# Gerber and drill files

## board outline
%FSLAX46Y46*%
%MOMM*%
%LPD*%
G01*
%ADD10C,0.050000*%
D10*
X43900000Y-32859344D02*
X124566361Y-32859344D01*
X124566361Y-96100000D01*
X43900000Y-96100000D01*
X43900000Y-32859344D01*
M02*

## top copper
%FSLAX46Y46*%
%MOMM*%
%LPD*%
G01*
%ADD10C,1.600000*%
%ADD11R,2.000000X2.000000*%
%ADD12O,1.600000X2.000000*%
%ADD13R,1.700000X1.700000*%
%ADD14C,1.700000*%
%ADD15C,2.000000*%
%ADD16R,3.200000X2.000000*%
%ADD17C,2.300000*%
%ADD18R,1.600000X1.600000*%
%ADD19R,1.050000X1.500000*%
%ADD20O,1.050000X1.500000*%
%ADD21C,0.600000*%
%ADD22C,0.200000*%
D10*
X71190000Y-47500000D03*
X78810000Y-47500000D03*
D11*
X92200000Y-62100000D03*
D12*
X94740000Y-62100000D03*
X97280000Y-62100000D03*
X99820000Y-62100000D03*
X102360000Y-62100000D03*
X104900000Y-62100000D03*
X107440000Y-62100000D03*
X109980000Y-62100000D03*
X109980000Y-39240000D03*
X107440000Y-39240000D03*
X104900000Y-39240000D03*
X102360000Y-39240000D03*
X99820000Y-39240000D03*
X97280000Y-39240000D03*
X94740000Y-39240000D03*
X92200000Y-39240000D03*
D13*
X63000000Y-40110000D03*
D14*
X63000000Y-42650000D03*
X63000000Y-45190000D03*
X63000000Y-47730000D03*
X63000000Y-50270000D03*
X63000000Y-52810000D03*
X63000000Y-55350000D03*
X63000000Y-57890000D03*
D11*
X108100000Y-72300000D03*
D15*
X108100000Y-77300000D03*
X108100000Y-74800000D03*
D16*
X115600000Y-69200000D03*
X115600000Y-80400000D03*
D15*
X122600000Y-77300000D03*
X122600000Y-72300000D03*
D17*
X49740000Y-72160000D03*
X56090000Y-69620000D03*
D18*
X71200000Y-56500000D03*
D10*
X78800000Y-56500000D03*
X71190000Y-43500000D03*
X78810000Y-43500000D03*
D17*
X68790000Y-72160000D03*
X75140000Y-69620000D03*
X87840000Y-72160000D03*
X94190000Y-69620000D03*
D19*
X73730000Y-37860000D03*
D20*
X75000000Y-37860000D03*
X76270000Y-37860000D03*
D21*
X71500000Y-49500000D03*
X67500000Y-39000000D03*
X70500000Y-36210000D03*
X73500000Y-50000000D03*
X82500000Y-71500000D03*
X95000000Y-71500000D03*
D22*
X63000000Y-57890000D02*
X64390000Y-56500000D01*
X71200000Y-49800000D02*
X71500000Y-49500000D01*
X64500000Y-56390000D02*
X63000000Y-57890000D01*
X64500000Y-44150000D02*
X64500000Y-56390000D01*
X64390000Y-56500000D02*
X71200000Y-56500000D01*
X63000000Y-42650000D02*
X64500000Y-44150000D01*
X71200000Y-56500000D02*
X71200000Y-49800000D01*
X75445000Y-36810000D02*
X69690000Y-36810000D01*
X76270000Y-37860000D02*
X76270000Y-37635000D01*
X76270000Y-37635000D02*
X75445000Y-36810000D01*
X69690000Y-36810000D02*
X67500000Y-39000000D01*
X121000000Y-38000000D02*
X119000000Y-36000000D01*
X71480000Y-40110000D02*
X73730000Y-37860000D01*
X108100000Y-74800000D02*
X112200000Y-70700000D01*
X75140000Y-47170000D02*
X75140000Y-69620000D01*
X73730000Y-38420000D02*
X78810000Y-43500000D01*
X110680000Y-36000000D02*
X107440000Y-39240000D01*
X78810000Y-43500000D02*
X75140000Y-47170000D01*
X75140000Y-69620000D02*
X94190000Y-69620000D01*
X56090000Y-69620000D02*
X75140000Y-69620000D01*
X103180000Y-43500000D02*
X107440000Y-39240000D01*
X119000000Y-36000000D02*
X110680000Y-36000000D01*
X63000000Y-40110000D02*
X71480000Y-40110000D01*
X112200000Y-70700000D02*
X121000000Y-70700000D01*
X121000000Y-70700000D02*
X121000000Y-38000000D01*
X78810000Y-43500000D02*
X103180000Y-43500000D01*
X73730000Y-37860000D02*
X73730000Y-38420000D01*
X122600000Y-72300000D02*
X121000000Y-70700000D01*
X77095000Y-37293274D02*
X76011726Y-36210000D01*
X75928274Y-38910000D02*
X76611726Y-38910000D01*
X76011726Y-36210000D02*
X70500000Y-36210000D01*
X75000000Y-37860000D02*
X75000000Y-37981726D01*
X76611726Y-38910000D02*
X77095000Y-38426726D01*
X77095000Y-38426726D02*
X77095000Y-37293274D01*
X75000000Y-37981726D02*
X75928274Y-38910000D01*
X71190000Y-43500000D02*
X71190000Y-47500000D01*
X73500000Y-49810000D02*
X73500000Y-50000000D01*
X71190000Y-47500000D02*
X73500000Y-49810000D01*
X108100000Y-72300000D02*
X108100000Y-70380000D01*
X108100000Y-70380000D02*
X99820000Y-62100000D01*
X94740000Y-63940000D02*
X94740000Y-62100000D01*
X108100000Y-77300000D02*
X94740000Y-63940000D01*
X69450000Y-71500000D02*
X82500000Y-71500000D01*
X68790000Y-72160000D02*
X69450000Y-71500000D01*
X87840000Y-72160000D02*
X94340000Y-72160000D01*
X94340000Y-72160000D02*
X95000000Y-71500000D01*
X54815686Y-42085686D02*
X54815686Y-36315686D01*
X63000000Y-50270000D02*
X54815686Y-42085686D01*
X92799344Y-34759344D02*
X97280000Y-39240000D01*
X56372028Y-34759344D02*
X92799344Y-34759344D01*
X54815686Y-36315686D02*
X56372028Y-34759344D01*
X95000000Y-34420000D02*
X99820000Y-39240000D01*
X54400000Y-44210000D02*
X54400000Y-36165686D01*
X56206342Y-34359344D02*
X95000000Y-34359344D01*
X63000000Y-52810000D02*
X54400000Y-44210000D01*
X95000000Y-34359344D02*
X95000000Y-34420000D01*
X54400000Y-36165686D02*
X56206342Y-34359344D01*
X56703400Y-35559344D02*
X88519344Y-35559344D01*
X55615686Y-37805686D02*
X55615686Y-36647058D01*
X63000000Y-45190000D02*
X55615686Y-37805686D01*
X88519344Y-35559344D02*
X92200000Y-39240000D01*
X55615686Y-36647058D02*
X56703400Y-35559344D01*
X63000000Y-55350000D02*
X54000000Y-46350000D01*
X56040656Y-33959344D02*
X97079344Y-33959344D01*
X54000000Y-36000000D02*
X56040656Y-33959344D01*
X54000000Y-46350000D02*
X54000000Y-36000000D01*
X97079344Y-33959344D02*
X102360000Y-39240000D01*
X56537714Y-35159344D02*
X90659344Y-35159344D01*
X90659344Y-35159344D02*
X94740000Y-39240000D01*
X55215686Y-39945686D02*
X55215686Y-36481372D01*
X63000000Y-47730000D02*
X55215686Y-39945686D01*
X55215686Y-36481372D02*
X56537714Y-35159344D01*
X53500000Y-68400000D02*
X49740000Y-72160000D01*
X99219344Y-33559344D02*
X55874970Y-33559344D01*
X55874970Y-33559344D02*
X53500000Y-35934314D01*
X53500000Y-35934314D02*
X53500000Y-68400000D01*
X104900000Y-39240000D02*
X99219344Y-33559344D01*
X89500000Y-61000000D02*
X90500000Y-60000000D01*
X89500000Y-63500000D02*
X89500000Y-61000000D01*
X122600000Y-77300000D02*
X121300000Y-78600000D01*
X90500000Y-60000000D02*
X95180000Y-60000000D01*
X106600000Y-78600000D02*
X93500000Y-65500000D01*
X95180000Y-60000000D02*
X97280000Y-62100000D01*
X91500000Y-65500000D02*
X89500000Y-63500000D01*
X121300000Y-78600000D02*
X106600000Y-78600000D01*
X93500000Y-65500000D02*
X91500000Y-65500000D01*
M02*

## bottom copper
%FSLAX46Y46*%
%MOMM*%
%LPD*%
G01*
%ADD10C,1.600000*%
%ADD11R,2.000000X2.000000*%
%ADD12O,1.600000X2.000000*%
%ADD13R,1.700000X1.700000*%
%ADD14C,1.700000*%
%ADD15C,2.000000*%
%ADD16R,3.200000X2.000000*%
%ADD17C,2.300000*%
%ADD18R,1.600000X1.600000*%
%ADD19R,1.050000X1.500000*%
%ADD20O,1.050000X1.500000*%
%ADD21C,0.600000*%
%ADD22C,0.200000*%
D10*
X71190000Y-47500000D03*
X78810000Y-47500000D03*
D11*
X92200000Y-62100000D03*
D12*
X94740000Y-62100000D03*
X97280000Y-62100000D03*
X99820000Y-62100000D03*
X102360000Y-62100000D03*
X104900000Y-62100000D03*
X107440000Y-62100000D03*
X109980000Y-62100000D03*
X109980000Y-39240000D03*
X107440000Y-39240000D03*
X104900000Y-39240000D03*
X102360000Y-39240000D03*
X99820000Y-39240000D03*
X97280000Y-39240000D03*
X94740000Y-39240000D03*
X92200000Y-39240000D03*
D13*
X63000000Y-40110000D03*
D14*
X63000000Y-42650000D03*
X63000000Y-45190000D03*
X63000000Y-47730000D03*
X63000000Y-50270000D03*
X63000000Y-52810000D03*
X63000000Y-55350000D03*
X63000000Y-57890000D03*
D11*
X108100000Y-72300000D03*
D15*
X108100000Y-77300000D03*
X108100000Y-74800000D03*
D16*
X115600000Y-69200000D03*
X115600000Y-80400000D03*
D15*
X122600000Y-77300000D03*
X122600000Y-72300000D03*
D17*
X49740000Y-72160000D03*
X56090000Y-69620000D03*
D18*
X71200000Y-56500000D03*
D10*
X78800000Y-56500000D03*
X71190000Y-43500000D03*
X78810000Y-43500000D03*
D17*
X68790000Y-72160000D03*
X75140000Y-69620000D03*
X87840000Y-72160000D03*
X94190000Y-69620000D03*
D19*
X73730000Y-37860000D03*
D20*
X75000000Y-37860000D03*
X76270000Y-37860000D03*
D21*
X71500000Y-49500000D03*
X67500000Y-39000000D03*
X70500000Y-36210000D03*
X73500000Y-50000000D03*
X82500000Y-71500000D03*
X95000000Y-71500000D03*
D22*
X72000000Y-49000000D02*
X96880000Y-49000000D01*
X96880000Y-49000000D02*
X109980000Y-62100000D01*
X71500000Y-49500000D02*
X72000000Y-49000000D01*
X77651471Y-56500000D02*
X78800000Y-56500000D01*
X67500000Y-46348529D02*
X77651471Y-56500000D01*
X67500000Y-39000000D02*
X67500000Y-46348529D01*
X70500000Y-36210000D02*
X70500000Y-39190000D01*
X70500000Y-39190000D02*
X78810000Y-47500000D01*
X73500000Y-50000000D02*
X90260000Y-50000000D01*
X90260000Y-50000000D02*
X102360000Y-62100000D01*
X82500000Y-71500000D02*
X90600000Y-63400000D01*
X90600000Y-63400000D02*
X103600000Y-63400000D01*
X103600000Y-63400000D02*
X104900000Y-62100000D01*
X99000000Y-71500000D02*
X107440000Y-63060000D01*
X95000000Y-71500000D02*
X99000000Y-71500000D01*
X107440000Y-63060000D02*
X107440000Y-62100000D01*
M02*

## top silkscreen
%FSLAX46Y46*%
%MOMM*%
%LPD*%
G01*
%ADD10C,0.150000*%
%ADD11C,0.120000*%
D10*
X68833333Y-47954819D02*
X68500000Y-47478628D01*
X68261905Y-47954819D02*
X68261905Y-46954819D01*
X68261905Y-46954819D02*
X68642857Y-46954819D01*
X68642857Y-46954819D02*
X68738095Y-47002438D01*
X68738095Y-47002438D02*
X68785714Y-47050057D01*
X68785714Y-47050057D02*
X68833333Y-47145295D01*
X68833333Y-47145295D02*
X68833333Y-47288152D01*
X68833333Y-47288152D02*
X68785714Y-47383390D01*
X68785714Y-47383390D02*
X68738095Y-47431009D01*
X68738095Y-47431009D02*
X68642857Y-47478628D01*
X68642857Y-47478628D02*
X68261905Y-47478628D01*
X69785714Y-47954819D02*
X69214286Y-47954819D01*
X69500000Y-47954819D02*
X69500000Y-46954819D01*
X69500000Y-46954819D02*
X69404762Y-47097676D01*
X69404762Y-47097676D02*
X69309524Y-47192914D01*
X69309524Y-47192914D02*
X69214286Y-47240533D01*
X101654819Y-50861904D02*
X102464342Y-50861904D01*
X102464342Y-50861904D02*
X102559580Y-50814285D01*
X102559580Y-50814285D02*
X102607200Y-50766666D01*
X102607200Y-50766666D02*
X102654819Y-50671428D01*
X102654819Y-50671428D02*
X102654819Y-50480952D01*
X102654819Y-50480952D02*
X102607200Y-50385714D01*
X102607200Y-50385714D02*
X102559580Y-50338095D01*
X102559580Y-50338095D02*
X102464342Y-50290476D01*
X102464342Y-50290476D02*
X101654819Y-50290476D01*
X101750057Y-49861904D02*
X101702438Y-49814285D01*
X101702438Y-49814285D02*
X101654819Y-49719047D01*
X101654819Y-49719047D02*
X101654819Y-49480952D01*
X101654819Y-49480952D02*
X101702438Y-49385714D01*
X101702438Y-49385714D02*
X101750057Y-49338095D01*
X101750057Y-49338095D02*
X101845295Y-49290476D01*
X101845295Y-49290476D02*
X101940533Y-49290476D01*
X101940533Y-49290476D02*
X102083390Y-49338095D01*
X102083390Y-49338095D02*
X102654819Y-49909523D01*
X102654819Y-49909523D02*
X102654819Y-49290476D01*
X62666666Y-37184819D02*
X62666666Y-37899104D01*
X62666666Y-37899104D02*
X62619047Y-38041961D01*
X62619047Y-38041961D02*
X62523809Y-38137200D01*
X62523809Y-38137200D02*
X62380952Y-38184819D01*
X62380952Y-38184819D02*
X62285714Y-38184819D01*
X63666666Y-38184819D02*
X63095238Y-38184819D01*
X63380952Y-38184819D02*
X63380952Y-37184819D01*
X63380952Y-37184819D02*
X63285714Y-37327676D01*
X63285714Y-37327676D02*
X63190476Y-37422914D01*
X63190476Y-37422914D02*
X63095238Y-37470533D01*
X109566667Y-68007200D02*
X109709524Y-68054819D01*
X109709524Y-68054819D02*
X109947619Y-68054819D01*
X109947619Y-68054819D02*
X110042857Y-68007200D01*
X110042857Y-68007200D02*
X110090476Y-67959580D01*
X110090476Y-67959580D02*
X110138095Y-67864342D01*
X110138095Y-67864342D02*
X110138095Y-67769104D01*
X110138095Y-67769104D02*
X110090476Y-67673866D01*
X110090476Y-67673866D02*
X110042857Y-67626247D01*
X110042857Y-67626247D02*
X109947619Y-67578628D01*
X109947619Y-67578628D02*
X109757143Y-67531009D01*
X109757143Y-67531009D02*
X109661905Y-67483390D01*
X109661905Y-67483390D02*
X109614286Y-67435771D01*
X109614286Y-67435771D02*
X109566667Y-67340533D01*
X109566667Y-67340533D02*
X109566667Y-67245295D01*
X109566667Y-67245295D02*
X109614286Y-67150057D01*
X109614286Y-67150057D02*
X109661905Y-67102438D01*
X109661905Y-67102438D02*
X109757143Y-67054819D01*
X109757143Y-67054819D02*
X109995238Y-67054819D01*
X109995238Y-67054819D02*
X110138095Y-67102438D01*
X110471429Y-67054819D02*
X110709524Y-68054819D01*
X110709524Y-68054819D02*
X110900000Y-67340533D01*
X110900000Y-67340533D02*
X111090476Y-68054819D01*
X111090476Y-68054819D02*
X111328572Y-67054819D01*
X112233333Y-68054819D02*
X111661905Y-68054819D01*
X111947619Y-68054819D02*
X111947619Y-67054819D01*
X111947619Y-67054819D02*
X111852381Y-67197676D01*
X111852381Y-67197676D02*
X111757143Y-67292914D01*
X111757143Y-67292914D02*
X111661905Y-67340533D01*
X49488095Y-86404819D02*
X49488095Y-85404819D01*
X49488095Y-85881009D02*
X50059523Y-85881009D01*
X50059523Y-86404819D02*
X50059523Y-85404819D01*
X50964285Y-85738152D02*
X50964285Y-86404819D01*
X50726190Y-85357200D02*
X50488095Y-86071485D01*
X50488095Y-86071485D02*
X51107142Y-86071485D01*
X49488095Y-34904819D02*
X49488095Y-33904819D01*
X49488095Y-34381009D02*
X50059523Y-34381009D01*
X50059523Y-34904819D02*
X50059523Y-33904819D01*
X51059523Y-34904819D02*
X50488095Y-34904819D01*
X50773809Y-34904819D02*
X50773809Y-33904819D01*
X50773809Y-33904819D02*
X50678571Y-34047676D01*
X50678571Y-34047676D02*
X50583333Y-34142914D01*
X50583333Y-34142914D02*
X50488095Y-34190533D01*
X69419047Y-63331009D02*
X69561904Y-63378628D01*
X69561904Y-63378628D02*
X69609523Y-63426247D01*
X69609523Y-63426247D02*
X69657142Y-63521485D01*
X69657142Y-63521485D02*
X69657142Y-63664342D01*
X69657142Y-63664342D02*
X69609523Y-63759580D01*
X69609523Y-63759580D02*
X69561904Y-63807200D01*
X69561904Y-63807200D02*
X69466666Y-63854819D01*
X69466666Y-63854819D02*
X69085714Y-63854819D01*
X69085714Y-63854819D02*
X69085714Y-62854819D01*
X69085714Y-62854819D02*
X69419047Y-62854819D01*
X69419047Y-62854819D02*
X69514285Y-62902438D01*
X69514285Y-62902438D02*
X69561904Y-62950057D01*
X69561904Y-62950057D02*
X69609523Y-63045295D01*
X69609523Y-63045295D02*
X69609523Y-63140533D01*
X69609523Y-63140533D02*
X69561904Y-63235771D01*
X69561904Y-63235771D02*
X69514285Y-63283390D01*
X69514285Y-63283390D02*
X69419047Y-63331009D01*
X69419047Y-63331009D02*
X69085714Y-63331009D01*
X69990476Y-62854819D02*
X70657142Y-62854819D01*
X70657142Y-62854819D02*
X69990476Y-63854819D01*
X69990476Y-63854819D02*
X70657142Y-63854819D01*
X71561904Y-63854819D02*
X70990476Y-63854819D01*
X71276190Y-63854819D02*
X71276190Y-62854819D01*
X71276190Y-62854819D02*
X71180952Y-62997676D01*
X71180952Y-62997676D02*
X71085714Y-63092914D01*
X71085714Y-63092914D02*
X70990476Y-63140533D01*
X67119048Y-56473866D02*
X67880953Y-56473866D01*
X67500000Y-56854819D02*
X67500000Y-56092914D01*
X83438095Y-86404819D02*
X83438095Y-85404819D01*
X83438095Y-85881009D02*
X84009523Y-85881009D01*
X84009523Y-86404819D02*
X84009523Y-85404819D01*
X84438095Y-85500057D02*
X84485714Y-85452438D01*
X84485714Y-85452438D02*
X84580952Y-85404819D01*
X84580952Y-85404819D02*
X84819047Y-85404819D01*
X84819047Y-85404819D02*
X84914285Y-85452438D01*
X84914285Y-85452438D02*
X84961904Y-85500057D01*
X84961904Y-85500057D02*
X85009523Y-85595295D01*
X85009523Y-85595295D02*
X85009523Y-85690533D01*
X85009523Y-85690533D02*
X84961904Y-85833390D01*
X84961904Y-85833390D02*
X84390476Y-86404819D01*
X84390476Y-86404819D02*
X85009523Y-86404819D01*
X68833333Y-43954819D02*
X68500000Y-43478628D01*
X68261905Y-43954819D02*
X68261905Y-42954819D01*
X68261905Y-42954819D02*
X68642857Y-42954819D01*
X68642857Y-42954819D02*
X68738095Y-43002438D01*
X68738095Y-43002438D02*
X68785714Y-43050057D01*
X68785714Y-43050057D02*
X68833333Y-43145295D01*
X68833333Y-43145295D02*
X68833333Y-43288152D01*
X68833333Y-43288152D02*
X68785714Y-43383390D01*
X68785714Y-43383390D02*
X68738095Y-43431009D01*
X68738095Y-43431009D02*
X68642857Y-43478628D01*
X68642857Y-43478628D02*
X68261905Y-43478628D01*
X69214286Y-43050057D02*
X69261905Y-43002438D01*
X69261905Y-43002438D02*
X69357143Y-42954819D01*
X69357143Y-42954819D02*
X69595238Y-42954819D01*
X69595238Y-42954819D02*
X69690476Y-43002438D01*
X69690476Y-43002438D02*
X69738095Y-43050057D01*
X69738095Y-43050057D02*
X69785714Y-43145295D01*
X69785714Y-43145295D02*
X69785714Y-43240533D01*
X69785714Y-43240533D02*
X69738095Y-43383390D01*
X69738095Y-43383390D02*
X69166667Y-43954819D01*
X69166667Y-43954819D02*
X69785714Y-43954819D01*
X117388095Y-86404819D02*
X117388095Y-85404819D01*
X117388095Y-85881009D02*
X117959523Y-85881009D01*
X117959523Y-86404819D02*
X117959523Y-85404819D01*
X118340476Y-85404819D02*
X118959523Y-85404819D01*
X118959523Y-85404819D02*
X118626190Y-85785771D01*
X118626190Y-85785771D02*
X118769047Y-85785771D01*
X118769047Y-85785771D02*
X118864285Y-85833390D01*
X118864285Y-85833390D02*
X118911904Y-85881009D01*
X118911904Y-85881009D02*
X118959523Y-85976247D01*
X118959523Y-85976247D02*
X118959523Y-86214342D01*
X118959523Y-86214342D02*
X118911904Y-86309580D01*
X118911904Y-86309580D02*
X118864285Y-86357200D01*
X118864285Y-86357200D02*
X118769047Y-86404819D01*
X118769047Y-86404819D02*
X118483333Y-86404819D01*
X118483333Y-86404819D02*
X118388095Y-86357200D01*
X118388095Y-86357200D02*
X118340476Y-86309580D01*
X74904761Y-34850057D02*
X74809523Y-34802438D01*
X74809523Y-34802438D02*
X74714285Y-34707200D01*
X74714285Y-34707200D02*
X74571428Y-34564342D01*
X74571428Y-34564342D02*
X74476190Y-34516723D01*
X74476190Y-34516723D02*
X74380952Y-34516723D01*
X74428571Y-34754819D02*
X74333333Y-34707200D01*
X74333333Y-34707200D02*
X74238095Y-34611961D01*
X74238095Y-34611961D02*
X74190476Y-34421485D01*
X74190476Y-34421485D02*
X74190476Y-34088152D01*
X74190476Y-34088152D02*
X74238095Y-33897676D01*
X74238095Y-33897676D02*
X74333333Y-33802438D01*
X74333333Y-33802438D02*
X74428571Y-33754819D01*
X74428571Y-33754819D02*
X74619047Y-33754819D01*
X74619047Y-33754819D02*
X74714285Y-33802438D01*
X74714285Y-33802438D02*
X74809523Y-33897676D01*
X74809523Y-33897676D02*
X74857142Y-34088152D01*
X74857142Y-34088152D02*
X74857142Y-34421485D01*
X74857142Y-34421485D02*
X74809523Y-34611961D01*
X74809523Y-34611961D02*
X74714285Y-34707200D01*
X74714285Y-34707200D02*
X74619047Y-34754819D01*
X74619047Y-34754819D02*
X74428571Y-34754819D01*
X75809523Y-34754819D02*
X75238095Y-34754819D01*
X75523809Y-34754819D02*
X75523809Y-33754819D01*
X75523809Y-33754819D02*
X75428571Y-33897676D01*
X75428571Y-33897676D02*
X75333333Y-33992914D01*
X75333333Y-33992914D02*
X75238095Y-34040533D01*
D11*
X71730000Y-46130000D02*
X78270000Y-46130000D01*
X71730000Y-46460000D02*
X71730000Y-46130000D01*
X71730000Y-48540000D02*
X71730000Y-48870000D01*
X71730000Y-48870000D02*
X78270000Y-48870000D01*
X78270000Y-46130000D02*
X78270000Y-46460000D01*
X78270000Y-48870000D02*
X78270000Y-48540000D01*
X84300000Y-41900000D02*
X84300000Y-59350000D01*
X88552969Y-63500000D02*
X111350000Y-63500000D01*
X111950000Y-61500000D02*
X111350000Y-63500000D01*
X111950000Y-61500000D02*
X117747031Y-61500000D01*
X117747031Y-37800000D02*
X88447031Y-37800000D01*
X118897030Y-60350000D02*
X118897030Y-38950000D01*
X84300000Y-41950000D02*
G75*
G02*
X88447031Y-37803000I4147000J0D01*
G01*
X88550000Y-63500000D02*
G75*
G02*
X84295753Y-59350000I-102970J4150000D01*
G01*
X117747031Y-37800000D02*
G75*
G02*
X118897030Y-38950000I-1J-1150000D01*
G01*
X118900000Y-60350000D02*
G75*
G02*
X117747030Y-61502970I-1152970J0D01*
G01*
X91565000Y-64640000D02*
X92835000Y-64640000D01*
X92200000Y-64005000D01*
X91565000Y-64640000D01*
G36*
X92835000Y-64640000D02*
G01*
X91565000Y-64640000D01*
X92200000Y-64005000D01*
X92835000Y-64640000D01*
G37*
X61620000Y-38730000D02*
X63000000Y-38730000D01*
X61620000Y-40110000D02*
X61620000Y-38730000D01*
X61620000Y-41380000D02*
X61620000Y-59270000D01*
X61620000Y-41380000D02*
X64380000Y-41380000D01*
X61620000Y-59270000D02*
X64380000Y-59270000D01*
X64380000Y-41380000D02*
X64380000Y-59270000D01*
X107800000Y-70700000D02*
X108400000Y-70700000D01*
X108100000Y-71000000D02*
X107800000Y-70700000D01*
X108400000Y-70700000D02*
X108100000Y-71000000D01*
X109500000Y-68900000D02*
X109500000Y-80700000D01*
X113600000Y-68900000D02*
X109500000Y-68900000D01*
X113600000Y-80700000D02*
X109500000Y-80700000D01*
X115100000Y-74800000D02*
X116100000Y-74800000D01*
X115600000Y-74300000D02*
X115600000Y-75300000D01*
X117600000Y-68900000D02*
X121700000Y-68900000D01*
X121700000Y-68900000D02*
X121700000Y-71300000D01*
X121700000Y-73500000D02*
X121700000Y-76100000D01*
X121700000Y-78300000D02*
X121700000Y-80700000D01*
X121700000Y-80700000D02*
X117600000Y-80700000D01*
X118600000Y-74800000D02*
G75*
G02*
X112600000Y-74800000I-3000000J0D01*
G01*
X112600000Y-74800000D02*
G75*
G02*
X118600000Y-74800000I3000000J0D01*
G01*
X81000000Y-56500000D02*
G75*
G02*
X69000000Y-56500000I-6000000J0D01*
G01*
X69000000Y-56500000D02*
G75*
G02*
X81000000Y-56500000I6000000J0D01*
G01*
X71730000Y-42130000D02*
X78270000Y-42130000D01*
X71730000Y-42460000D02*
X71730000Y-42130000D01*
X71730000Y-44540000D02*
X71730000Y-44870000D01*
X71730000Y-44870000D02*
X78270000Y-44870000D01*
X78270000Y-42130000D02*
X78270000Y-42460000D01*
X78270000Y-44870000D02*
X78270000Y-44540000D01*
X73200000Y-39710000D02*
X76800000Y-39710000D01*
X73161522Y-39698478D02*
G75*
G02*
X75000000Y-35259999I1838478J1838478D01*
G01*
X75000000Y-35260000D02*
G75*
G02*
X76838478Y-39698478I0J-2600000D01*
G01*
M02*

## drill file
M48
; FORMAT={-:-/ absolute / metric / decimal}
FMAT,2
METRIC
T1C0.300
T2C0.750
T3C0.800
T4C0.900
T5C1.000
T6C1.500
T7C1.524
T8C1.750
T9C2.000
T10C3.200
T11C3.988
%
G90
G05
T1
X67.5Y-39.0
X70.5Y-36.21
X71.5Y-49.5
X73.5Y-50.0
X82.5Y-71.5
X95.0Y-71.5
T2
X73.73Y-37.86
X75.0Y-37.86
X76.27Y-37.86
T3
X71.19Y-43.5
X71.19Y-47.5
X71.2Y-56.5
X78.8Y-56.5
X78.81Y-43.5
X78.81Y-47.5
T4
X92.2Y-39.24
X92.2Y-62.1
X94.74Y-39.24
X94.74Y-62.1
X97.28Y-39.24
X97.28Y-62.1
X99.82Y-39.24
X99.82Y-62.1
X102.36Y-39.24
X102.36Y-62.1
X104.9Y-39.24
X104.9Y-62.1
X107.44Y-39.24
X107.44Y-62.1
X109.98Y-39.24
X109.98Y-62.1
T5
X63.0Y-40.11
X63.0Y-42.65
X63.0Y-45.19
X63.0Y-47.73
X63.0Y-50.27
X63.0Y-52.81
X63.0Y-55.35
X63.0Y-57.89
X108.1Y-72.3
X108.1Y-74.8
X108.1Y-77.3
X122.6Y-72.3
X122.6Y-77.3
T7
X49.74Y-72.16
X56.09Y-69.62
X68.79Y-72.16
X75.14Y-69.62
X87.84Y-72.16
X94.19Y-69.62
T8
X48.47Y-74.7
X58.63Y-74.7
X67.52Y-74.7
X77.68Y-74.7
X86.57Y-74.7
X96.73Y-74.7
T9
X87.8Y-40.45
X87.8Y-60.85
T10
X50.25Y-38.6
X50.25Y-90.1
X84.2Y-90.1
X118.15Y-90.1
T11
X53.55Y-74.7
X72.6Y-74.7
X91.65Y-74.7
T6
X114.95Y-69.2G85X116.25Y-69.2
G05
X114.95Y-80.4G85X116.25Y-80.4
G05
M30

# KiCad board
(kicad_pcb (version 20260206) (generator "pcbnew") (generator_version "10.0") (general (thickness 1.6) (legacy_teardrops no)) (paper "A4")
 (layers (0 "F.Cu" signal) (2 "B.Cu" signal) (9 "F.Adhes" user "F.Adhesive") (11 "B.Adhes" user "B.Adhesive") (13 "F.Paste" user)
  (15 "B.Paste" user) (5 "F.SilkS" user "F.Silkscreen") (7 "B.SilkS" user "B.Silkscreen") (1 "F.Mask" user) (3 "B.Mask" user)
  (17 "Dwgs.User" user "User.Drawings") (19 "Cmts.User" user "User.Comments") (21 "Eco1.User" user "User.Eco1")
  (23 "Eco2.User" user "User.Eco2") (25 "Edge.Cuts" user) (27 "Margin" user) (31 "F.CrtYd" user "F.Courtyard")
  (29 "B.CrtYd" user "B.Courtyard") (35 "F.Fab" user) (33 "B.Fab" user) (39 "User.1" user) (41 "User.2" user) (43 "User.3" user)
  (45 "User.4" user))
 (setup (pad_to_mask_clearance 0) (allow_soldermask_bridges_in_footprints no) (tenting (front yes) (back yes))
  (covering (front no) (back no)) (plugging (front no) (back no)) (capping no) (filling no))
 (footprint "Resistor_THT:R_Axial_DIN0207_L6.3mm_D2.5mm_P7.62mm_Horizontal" (layer "F.Cu") (at 71.19 47.5)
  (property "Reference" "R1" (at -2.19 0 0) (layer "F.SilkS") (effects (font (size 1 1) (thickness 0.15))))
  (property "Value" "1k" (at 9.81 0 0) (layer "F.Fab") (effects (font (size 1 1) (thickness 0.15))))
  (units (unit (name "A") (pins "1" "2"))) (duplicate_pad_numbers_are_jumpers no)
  (fp_line (start 0.54 -1.37) (end 7.08 -1.37) (stroke (width 0.12) (type solid)) (layer "F.SilkS"))
  (fp_line (start 0.54 -1.04) (end 0.54 -1.37) (stroke (width 0.12) (type solid)) (layer "F.SilkS"))
  (fp_line (start 0.54 1.04) (end 0.54 1.37) (stroke (width 0.12) (type solid)) (layer "F.SilkS"))
  (fp_line (start 0.54 1.37) (end 7.08 1.37) (stroke (width 0.12) (type solid)) (layer "F.SilkS"))
  (fp_line (start 7.08 -1.37) (end 7.08 -1.04) (stroke (width 0.12) (type solid)) (layer "F.SilkS"))
  (fp_line (start 7.08 1.37) (end 7.08 1.04) (stroke (width 0.12) (type solid)) (layer "F.SilkS"))
  (pad "1" thru_hole circle (at 0 0) (size 1.6 1.6) (drill 0.8) (layers "*.Cu" "*.Mask") (remove_unused_layers no) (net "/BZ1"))
  (pad "2" thru_hole circle (at 7.62 0) (size 1.6 1.6) (drill 0.8) (layers "*.Cu" "*.Mask") (remove_unused_layers no) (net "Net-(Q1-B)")))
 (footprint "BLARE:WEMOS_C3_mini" (layer "F.Cu") (at 92.2 62.1 90)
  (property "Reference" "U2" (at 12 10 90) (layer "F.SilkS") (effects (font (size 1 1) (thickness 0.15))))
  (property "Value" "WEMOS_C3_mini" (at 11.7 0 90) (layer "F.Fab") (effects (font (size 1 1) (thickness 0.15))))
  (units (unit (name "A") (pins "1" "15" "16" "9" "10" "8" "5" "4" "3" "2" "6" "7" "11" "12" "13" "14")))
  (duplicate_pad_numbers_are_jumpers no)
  (fp_line (start 20.2 -7.9) (end 2.75 -7.9) (stroke (width 0.12) (type solid)) (layer "F.SilkS"))
  (fp_line (start -1.4 -3.647031) (end -1.4 19.15) (stroke (width 0.12) (type solid)) (layer "F.SilkS"))
  (fp_line (start 0.6 19.75) (end -1.4 19.15) (stroke (width 0.12) (type default)) (layer "F.SilkS"))
  (fp_line (start 0.6 19.75) (end 0.6 25.547031) (stroke (width 0.12) (type solid)) (layer "F.SilkS"))
  (fp_line (start 24.3 25.547031) (end 24.3 -3.752969) (stroke (width 0.12) (type solid)) (layer "F.SilkS"))
  (fp_line (start 1.75 26.69703) (end 23.15 26.69703) (stroke (width 0.12) (type solid)) (layer "F.SilkS"))
  (fp_arc (start 20.15 -7.9) (mid 23.082383 -6.685361) (end 24.297 -3.752969) (stroke (width 0.12) (type solid)) (layer "F.SilkS"))
  (fp_arc (start -1.4 -3.65) (mid -0.221578 -6.651732) (end 2.75 -7.904246) (stroke (width 0.12) (type solid)) (layer "F.SilkS"))
  (fp_arc (start 24.3 25.547031) (mid 23.963172 26.360203) (end 23.15 26.69703) (stroke (width 0.12) (type solid)) (layer "F.SilkS"))
  (fp_arc (start 1.75 26.7) (mid 0.934727 26.362303) (end 0.59703 25.54703) (stroke (width 0.12) (type solid)) (layer "F.SilkS"))
  (fp_poly (pts (xy -2.54 -0.635) (xy -2.54 0.635) (xy -1.905 0)) (stroke (width 0.12) (type solid)) (fill yes) (layer "F.SilkS"))
  (pad "" np_thru_hole circle (at 1.25 -4.4 90) (size 3 3) (drill 2) (layers "*.Mask"))
  (pad "" np_thru_hole circle (at 21.65 -4.4 90) (size 3 3) (drill 2) (layers "*.Mask"))
  (pad "1" thru_hole rect (at 0 0 90) (size 2 2) (drill 0.9) (layers "*.Cu" "*.Mask") (remove_unused_layers no)
   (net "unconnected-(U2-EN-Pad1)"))
  (pad "2" thru_hole oval (at 0 2.54 90) (size 2 1.6) (drill 0.9) (layers "*.Cu" "*.Mask") (remove_unused_layers no) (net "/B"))
  (pad "3" thru_hole oval (at 0 5.08 90) (size 2 1.6) (drill 0.9) (layers "*.Cu" "*.Mask") (remove_unused_layers no) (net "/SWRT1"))
  (pad "4" thru_hole oval (at 0 7.62 90) (size 2 1.6) (drill 0.9) (layers "*.Cu" "*.Mask") (remove_unused_layers no) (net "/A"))
  (pad "5" thru_hole oval (at 0 10.16 90) (size 2 1.6) (drill 0.9) (layers "*.Cu" "*.Mask") (remove_unused_layers no) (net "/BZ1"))
  (pad "6" thru_hole oval (at 0 12.7 90) (size 2 1.6) (drill 0.9) (layers "*.Cu" "*.Mask") (remove_unused_layers no) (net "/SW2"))
  (pad "7" thru_hole oval (at 0 15.24 90) (size 2 1.6) (drill 0.9) (layers "*.Cu" "*.Mask") (remove_unused_layers no) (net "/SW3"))
  (pad "8" thru_hole oval (at 0 17.78 90) (size 2 1.6) (drill 0.9) (layers "*.Cu" "*.Mask") (remove_unused_layers no) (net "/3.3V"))
  (pad "9" thru_hole oval (at 22.86 17.78 90) (size 2 1.6) (drill 0.9) (layers "*.Cu" "*.Mask") (remove_unused_layers no)
   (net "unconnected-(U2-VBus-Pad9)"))
  (pad "10" thru_hole oval (at 22.86 15.24 90) (size 2 1.6) (drill 0.9) (layers "*.Cu" "*.Mask") (remove_unused_layers no) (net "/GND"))
  (pad "11" thru_hole oval (at 22.86 12.7 90) (size 2 1.6) (drill 0.9) (layers "*.Cu" "*.Mask") (remove_unused_layers no) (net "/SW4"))
  (pad "12" thru_hole oval (at 22.86 10.16 90) (size 2 1.6) (drill 0.9) (layers "*.Cu" "*.Mask") (remove_unused_layers no) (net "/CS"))
  (pad "13" thru_hole oval (at 22.86 7.62 90) (size 2 1.6) (drill 0.9) (layers "*.Cu" "*.Mask") (remove_unused_layers no) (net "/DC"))
  (pad "14" thru_hole oval (at 22.86 5.08 90) (size 2 1.6) (drill 0.9) (layers "*.Cu" "*.Mask") (remove_unused_layers no) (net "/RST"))
  (pad "15" thru_hole oval (at 22.86 2.54 90) (size 2 1.6) (drill 0.9) (layers "*.Cu" "*.Mask") (remove_unused_layers no) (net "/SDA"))
  (pad "16" thru_hole oval (at 22.86 0 90) (size 2 1.6) (drill 0.9) (layers "*.Cu" "*.Mask") (remove_unused_layers no) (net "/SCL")))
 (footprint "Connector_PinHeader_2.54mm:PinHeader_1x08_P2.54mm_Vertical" (layer "F.Cu") (at 63 40.11)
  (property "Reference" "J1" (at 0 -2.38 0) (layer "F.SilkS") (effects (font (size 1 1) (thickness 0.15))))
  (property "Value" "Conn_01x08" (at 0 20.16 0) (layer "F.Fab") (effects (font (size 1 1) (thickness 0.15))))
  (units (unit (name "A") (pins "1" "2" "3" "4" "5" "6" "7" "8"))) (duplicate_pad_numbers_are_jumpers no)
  (fp_line (start -1.38 -1.38) (end 0 -1.38) (stroke (width 0.12) (type solid)) (layer "F.SilkS"))
  (fp_line (start -1.38 0) (end -1.38 -1.38) (stroke (width 0.12) (type solid)) (layer "F.SilkS"))
  (fp_line (start -1.38 1.27) (end -1.38 19.16) (stroke (width 0.12) (type solid)) (layer "F.SilkS"))
  (fp_line (start -1.38 1.27) (end 1.38 1.27) (stroke (width 0.12) (type solid)) (layer "F.SilkS"))
  (fp_line (start -1.38 19.16) (end 1.38 19.16) (stroke (width 0.12) (type solid)) (layer "F.SilkS"))
  (fp_line (start 1.38 1.27) (end 1.38 19.16) (stroke (width 0.12) (type solid)) (layer "F.SilkS"))
  (pad "1" thru_hole rect (at 0 0) (size 1.7 1.7) (drill 1) (layers "*.Cu" "*.Mask") (remove_unused_layers no) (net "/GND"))
  (pad "2" thru_hole circle (at 0 2.54) (size 1.7 1.7) (drill 1) (layers "*.Cu" "*.Mask") (remove_unused_layers no) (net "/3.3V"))
  (pad "3" thru_hole circle (at 0 5.08) (size 1.7 1.7) (drill 1) (layers "*.Cu" "*.Mask") (remove_unused_layers no) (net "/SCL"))
  (pad "4" thru_hole circle (at 0 7.62) (size 1.7 1.7) (drill 1) (layers "*.Cu" "*.Mask") (remove_unused_layers no) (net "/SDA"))
  (pad "5" thru_hole circle (at 0 10.16) (size 1.7 1.7) (drill 1) (layers "*.Cu" "*.Mask") (remove_unused_layers no) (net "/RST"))
  (pad "6" thru_hole circle (at 0 12.7) (size 1.7 1.7) (drill 1) (layers "*.Cu" "*.Mask") (remove_unused_layers no) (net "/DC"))
  (pad "7" thru_hole circle (at 0 15.24) (size 1.7 1.7) (drill 1) (layers "*.Cu" "*.Mask") (remove_unused_layers no) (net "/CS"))
  (pad "8" thru_hole circle (at 0 17.78) (size 1.7 1.7) (drill 1) (layers "*.Cu" "*.Mask") (remove_unused_layers no) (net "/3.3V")))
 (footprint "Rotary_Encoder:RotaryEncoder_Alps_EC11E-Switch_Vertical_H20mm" (layer "F.Cu") (at 108.1 72.3)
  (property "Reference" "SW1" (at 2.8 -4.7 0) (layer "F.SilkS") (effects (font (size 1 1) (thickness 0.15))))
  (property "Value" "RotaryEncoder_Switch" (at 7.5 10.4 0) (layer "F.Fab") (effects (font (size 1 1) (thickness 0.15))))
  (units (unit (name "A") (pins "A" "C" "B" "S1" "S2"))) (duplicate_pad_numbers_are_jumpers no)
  (fp_line (start -0.3 -1.6) (end 0.3 -1.6) (stroke (width 0.12) (type solid)) (layer "F.SilkS"))
  (fp_line (start 0 -1.3) (end -0.3 -1.6) (stroke (width 0.12) (type solid)) (layer "F.SilkS"))
  (fp_line (start 0.3 -1.6) (end 0 -1.3) (stroke (width 0.12) (type solid)) (layer "F.SilkS"))
  (fp_line (start 1.4 -3.4) (end 1.4 8.4) (stroke (width 0.12) (type solid)) (layer "F.SilkS"))
  (fp_line (start 5.5 -3.4) (end 1.4 -3.4) (stroke (width 0.12) (type solid)) (layer "F.SilkS"))
  (fp_line (start 5.5 8.4) (end 1.4 8.4) (stroke (width 0.12) (type solid)) (layer "F.SilkS"))
  (fp_line (start 7 2.5) (end 8 2.5) (stroke (width 0.12) (type solid)) (layer "F.SilkS"))
  (fp_line (start 7.5 2) (end 7.5 3) (stroke (width 0.12) (type solid)) (layer "F.SilkS"))
  (fp_line (start 9.5 -3.4) (end 13.6 -3.4) (stroke (width 0.12) (type solid)) (layer "F.SilkS"))
  (fp_line (start 13.6 -3.4) (end 13.6 -1) (stroke (width 0.12) (type solid)) (layer "F.SilkS"))
  (fp_line (start 13.6 1.2) (end 13.6 3.8) (stroke (width 0.12) (type solid)) (layer "F.SilkS"))
  (fp_line (start 13.6 6) (end 13.6 8.4) (stroke (width 0.12) (type solid)) (layer "F.SilkS"))
  (fp_line (start 13.6 8.4) (end 9.5 8.4) (stroke (width 0.12) (type solid)) (layer "F.SilkS"))
  (fp_circle (center 7.5 2.5) (end 10.5 2.5) (stroke (width 0.12) (type solid)) (fill no) (layer "F.SilkS"))
  (pad "A" thru_hole rect (at 0 0) (size 2 2) (drill 1) (layers "*.Cu" "*.Mask") (remove_unused_layers no) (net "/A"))
  (pad "B" thru_hole circle (at 0 5) (size 2 2) (drill 1) (layers "*.Cu" "*.Mask") (remove_unused_layers no) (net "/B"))
  (pad "C" thru_hole circle (at 0 2.5) (size 2 2) (drill 1) (layers "*.Cu" "*.Mask") (remove_unused_layers no) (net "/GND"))
  (pad "MP" thru_hole rect (at 7.5 -3.1) (size 3.2 2) (drill oval 2.8 1.5) (layers "*.Cu" "*.Mask") (remove_unused_layers no))
  (pad "MP" thru_hole rect (at 7.5 8.1) (size 3.2 2) (drill oval 2.8 1.5) (layers "*.Cu" "*.Mask") (remove_unused_layers no))
  (pad "S1" thru_hole circle (at 14.5 5) (size 2 2) (drill 1) (layers "*.Cu" "*.Mask") (remove_unused_layers no) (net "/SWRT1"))
  (pad "S2" thru_hole circle (at 14.5 0) (size 2 2) (drill 1) (layers "*.Cu" "*.Mask") (remove_unused_layers no) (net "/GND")))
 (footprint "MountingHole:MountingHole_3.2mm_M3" (layer "F.Cu") (at 50.25 90.1)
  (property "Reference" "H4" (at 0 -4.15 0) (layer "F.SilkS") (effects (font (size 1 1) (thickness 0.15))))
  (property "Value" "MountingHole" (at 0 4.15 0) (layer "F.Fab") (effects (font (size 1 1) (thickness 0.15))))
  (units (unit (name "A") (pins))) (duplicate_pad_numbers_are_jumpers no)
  (pad "" np_thru_hole circle (at 0 0) (size 3.2 3.2) (drill 3.2) (layers "*.Cu" "*.Mask")))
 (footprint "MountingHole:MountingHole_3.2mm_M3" (layer "F.Cu") (at 50.25 38.6)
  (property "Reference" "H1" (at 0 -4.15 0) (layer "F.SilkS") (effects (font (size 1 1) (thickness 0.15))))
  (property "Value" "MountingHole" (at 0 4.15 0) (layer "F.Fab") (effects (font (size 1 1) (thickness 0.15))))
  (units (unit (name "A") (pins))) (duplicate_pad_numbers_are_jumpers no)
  (pad "" np_thru_hole circle (at 0 0) (size 3.2 3.2) (drill 3.2) (layers "*.Cu" "*.Mask")))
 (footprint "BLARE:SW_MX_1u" (layer "F.Cu") (at 53.55 74.7)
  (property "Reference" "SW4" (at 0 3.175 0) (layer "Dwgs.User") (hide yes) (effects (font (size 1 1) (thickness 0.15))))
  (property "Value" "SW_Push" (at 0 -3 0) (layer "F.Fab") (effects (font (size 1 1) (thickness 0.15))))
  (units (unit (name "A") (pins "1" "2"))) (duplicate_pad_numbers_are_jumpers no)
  (pad "" np_thru_hole circle (at -5.08 0) (size 1.75 1.75) (drill 1.75) (layers "*.Cu" "*.Mask"))
  (pad "" np_thru_hole circle (at 0 0) (size 3.9878 3.9878) (drill 3.9878) (layers "*.Cu" "*.Mask"))
  (pad "" np_thru_hole circle (at 5.08 0) (size 1.75 1.75) (drill 1.75) (layers "*.Cu" "*.Mask"))
  (pad "1" thru_hole circle (at -3.81 -2.54) (size 2.3 2.3) (drill 1.524) (layers "*.Cu" "B.Mask") (remove_unused_layers no) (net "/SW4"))
  (pad "2" thru_hole circle (at 2.54 -5.08) (size 2.3 2.3) (drill 1.524) (layers "*.Cu" "B.Mask") (remove_unused_layers no) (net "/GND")))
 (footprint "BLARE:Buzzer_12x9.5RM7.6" (layer "F.Cu") (at 75 56.5)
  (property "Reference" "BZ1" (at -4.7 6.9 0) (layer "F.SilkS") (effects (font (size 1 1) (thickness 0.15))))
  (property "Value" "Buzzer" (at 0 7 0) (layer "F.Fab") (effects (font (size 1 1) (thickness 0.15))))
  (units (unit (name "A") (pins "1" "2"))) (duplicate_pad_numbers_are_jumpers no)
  (fp_circle (center 0 0) (end 6 0) (stroke (width 0.12) (type solid)) (fill no) (layer "F.SilkS"))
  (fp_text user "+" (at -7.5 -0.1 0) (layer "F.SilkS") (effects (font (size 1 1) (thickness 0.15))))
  (pad "1" thru_hole rect (at -3.8 0) (size 1.6 1.6) (drill 0.8) (layers "*.Cu" "*.Mask") (remove_unused_layers no) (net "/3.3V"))
  (pad "2" thru_hole circle (at 3.8 0) (size 1.6 1.6) (drill 0.8) (layers "*.Cu" "*.Mask") (remove_unused_layers no) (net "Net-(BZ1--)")))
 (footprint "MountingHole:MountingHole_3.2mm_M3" (layer "F.Cu") (at 84.2 90.1)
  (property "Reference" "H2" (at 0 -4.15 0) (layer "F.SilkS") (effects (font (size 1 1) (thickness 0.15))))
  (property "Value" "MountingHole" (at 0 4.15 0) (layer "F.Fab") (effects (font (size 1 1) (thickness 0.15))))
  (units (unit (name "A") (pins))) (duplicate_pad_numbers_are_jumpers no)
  (pad "" np_thru_hole circle (at 0 0) (size 3.2 3.2) (drill 3.2) (layers "*.Cu" "*.Mask")))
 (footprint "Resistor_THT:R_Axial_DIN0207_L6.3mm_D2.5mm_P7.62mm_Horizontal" (layer "F.Cu") (at 71.19 43.5)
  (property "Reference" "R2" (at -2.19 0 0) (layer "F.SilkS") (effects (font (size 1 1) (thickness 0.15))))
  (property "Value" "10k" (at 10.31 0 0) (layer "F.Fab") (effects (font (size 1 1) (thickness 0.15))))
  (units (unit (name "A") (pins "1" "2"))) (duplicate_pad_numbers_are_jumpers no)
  (fp_line (start 0.54 -1.37) (end 7.08 -1.37) (stroke (width 0.12) (type solid)) (layer "F.SilkS"))
  (fp_line (start 0.54 -1.04) (end 0.54 -1.37) (stroke (width 0.12) (type solid)) (layer "F.SilkS"))
  (fp_line (start 0.54 1.04) (end 0.54 1.37) (stroke (width 0.12) (type solid)) (layer "F.SilkS"))
  (fp_line (start 0.54 1.37) (end 7.08 1.37) (stroke (width 0.12) (type solid)) (layer "F.SilkS"))
  (fp_line (start 7.08 -1.37) (end 7.08 -1.04) (stroke (width 0.12) (type solid)) (layer "F.SilkS"))
  (fp_line (start 7.08 1.37) (end 7.08 1.04) (stroke (width 0.12) (type solid)) (layer "F.SilkS"))
  (pad "1" thru_hole circle (at 0 0) (size 1.6 1.6) (drill 0.8) (layers "*.Cu" "*.Mask") (remove_unused_layers no) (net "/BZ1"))
  (pad "2" thru_hole circle (at 7.62 0) (size 1.6 1.6) (drill 0.8) (layers "*.Cu" "*.Mask") (remove_unused_layers no) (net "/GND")))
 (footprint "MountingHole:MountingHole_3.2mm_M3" (layer "F.Cu") (at 118.15 90.1)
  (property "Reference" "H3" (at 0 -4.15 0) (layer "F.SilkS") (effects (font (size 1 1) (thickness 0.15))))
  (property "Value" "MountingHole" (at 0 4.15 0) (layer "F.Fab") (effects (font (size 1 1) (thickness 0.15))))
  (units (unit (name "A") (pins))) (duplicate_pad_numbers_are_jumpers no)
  (pad "" np_thru_hole circle (at 0 0) (size 3.2 3.2) (drill 3.2) (layers "*.Cu" "*.Mask")))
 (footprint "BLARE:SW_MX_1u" (layer "F.Cu") (at 72.6 74.7)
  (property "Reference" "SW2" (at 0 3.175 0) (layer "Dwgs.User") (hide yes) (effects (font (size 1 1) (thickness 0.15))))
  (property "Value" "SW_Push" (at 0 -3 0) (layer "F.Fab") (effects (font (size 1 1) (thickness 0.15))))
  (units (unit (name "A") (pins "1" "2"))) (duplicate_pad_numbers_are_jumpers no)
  (pad "" np_thru_hole circle (at -5.08 0) (size 1.75 1.75) (drill 1.75) (layers "*.Cu" "*.Mask"))
  (pad "" np_thru_hole circle (at 0 0) (size 3.9878 3.9878) (drill 3.9878) (layers "*.Cu" "*.Mask"))
  (pad "" np_thru_hole circle (at 5.08 0) (size 1.75 1.75) (drill 1.75) (layers "*.Cu" "*.Mask"))
  (pad "1" thru_hole circle (at -3.81 -2.54) (size 2.3 2.3) (drill 1.524) (layers "*.Cu" "B.Mask") (remove_unused_layers no) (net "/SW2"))
  (pad "2" thru_hole circle (at 2.54 -5.08) (size 2.3 2.3) (drill 1.524) (layers "*.Cu" "B.Mask") (remove_unused_layers no) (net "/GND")))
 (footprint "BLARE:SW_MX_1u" (layer "F.Cu") (at 91.65 74.7)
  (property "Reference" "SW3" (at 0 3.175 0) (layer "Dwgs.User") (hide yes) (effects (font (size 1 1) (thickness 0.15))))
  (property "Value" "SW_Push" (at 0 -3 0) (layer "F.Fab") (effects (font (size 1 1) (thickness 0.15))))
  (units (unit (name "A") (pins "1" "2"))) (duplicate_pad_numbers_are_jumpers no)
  (pad "" np_thru_hole circle (at -5.08 0) (size 1.75 1.75) (drill 1.75) (layers "*.Cu" "*.Mask"))
  (pad "" np_thru_hole circle (at 0 0) (size 3.9878 3.9878) (drill 3.9878) (layers "*.Cu" "*.Mask"))
  (pad "" np_thru_hole circle (at 5.08 0) (size 1.75 1.75) (drill 1.75) (layers "*.Cu" "*.Mask"))
  (pad "1" thru_hole circle (at -3.81 -2.54) (size 2.3 2.3) (drill 1.524) (layers "*.Cu" "B.Mask") (remove_unused_layers no) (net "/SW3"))
  (pad "2" thru_hole circle (at 2.54 -5.08) (size 2.3 2.3) (drill 1.524) (layers "*.Cu" "B.Mask") (remove_unused_layers no) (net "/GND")))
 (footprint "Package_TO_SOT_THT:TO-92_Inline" (layer "F.Cu") (at 73.73 37.86)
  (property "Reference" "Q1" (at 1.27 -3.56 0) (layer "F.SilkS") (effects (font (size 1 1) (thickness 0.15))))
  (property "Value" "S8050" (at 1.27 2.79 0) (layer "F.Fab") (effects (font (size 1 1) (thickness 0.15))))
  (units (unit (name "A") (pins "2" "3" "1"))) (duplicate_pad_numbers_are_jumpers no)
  (fp_line (start -0.53 1.85) (end 3.07 1.85) (stroke (width 0.12) (type solid)) (layer "F.SilkS"))
  (fp_arc (start -0.568478 1.838478) (mid -1.132087 -0.994977) (end 1.27 -2.6) (stroke (width 0.12) (type solid)) (layer "F.SilkS"))
  (fp_arc (start 1.27 -2.6) (mid 3.672087 -0.994977) (end 3.108478 1.838478) (stroke (width 0.12) (type solid)) (layer "F.SilkS"))
  (pad "1" thru_hole rect (at 0 0) (size 1.05 1.5) (drill 0.75) (layers "*.Cu" "*.Mask") (remove_unused_layers no) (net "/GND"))
  (pad "2" thru_hole oval (at 1.27 0) (size 1.05 1.5) (drill 0.75) (layers "*.Cu" "*.Mask") (remove_unused_layers no) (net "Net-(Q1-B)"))
  (pad "3" thru_hole oval (at 2.54 0) (size 1.05 1.5) (drill 0.75) (layers "*.Cu" "*.Mask") (remove_unused_layers no) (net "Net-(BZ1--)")))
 (gr_rect (start 43.9 32.859344) (end 124.566361 96.1) (stroke (width 0.05) (type default)) (fill no) (layer "Edge.Cuts"))
 (segment (start 63 57.89) (end 64.39 56.5) (width 0.2) (layer "F.Cu") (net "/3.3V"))
 (segment (start 71.2 49.8) (end 71.5 49.5) (width 0.2) (layer "F.Cu") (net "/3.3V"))
 (segment (start 64.5 56.39) (end 63 57.89) (width 0.2) (layer "F.Cu") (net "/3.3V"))
 (segment (start 64.5 44.15) (end 64.5 56.39) (width 0.2) (layer "F.Cu") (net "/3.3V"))
 (segment (start 64.39 56.5) (end 71.2 56.5) (width 0.2) (layer "F.Cu") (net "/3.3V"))
 (segment (start 63 42.65) (end 64.5 44.15) (width 0.2) (layer "F.Cu") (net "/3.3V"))
 (segment (start 71.2 56.5) (end 71.2 49.8) (width 0.2) (layer "F.Cu") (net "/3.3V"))
 (via (at 71.5 49.5) (size 0.6) (drill 0.3) (layers "F.Cu" "B.Cu") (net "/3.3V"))
 (segment (start 72 49) (end 96.88 49) (width 0.2) (layer "B.Cu") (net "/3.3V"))
 (segment (start 96.88 49) (end 109.98 62.1) (width 0.2) (layer "B.Cu") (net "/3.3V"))
 (segment (start 71.5 49.5) (end 72 49) (width 0.2) (layer "B.Cu") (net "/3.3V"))
 (segment (start 75.445 36.81) (end 69.69 36.81) (width 0.2) (layer "F.Cu") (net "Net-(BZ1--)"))
 (segment (start 76.27 37.86) (end 76.27 37.635) (width 0.2) (layer "F.Cu") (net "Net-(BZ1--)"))
 (segment (start 76.27 37.635) (end 75.445 36.81) (width 0.2) (layer "F.Cu") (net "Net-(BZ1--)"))
 (segment (start 69.69 36.81) (end 67.5 39) (width 0.2) (layer "F.Cu") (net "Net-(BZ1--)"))
 (via (at 67.5 39) (size 0.6) (drill 0.3) (layers "F.Cu" "B.Cu") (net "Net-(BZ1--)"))
 (segment (start 77.651471 56.5) (end 78.8 56.5) (width 0.2) (layer "B.Cu") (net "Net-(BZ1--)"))
 (segment (start 67.5 46.348529) (end 77.651471 56.5) (width 0.2) (layer "B.Cu") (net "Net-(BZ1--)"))
 (segment (start 67.5 39) (end 67.5 46.348529) (width 0.2) (layer "B.Cu") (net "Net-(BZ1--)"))
 (segment (start 121 38) (end 119 36) (width 0.2) (layer "F.Cu") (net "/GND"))
 (segment (start 71.48 40.11) (end 73.73 37.86) (width 0.2) (layer "F.Cu") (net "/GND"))
 (segment (start 108.1 74.8) (end 112.2 70.7) (width 0.2) (layer "F.Cu") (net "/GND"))
 (segment (start 75.14 47.17) (end 75.14 69.62) (width 0.2) (layer "F.Cu") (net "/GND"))
 (segment (start 73.73 38.42) (end 78.81 43.5) (width 0.2) (layer "F.Cu") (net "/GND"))
 (segment (start 110.68 36) (end 107.44 39.24) (width 0.2) (layer "F.Cu") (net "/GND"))
 (segment (start 78.81 43.5) (end 75.14 47.17) (width 0.2) (layer "F.Cu") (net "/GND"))
 (segment (start 75.14 69.62) (end 94.19 69.62) (width 0.2) (layer "F.Cu") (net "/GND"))
 (segment (start 56.09 69.62) (end 75.14 69.62) (width 0.2) (layer "F.Cu") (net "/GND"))
 (segment (start 103.18 43.5) (end 107.44 39.24) (width 0.2) (layer "F.Cu") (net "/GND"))
 (segment (start 119 36) (end 110.68 36) (width 0.2) (layer "F.Cu") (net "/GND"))
 (segment (start 63 40.11) (end 71.48 40.11) (width 0.2) (layer "F.Cu") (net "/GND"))
 (segment (start 112.2 70.7) (end 121 70.7) (width 0.2) (layer "F.Cu") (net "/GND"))
 (segment (start 121 70.7) (end 121 38) (width 0.2) (layer "F.Cu") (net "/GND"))
 (segment (start 78.81 43.5) (end 103.18 43.5) (width 0.2) (layer "F.Cu") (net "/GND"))
 (segment (start 73.73 37.86) (end 73.73 38.42) (width 0.2) (layer "F.Cu") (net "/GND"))
 (segment (start 122.6 72.3) (end 121 70.7) (width 0.2) (layer "F.Cu") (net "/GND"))
 (segment (start 77.095 37.293274) (end 76.011726 36.21) (width 0.2) (layer "F.Cu") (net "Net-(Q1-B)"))
 (segment (start 75.928274 38.91) (end 76.611726 38.91) (width 0.2) (layer "F.Cu") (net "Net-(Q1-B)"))
 (segment (start 76.011726 36.21) (end 70.5 36.21) (width 0.2) (layer "F.Cu") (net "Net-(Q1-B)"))
 (segment (start 75 37.86) (end 75 37.981726) (width 0.2) (layer "F.Cu") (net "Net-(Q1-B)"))
 (segment (start 76.611726 38.91) (end 77.095 38.426726) (width 0.2) (layer "F.Cu") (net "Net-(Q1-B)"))
 (segment (start 77.095 38.426726) (end 77.095 37.293274) (width 0.2) (layer "F.Cu") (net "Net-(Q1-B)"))
 (segment (start 75 37.981726) (end 75.928274 38.91) (width 0.2) (layer "F.Cu") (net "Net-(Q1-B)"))
 (via (at 70.5 36.21) (size 0.6) (drill 0.3) (layers "F.Cu" "B.Cu") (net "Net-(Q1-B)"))
 (segment (start 70.5 36.21) (end 70.5 39.19) (width 0.2) (layer "B.Cu") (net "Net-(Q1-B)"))
 (segment (start 70.5 39.19) (end 78.81 47.5) (width 0.2) (layer "B.Cu") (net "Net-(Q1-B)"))
 (segment (start 71.19 43.5) (end 71.19 47.5) (width 0.2) (layer "F.Cu") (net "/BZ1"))
 (segment (start 73.5 49.81) (end 73.5 50) (width 0.2) (layer "F.Cu") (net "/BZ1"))
 (segment (start 71.19 47.5) (end 73.5 49.81) (width 0.2) (layer "F.Cu") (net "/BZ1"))
 (via (at 73.5 50) (size 0.6) (drill 0.3) (layers "F.Cu" "B.Cu") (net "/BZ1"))
 (segment (start 73.5 50) (end 90.26 50) (width 0.2) (layer "B.Cu") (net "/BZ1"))
 (segment (start 90.26 50) (end 102.36 62.1) (width 0.2) (layer "B.Cu") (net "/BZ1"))
 (segment (start 108.1 72.3) (end 108.1 70.38) (width 0.2) (layer "F.Cu") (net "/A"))
 (segment (start 108.1 70.38) (end 99.82 62.1) (width 0.2) (layer "F.Cu") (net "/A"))
 (segment (start 94.74 63.94) (end 94.74 62.1) (width 0.2) (layer "F.Cu") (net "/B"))
 (segment (start 108.1 77.3) (end 94.74 63.94) (width 0.2) (layer "F.Cu") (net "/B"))
 (segment (start 69.45 71.5) (end 82.5 71.5) (width 0.2) (layer "F.Cu") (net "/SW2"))
 (segment (start 68.79 72.16) (end 69.45 71.5) (width 0.2) (layer "F.Cu") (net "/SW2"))
 (via (at 82.5 71.5) (size 0.6) (drill 0.3) (layers "F.Cu" "B.Cu") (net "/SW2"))
 (segment (start 82.5 71.5) (end 90.6 63.4) (width 0.2) (layer "B.Cu") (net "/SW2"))
 (segment (start 90.6 63.4) (end 103.6 63.4) (width 0.2) (layer "B.Cu") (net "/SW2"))
 (segment (start 103.6 63.4) (end 104.9 62.1) (width 0.2) (layer "B.Cu") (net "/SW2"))
 (segment (start 87.84 72.16) (end 94.34 72.16) (width 0.2) (layer "F.Cu") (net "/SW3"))
 (segment (start 94.34 72.16) (end 95 71.5) (width 0.2) (layer "F.Cu") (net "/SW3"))
 (via (at 95 71.5) (size 0.6) (drill 0.3) (layers "F.Cu" "B.Cu") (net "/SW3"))
 (segment (start 99 71.5) (end 107.44 63.06) (width 0.2) (layer "B.Cu") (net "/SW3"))
 (segment (start 95 71.5) (end 99 71.5) (width 0.2) (layer "B.Cu") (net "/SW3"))
 (segment (start 107.44 63.06) (end 107.44 62.1) (width 0.2) (layer "B.Cu") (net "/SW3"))
 (segment (start 54.815686 42.085686) (end 54.815686 36.315686) (width 0.2) (layer "F.Cu") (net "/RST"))
 (segment (start 63 50.27) (end 54.815686 42.085686) (width 0.2) (layer "F.Cu") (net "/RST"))
 (segment (start 92.799344 34.759344) (end 97.28 39.24) (width 0.2) (layer "F.Cu") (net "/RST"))
 (segment (start 56.372028 34.759344) (end 92.799344 34.759344) (width 0.2) (layer "F.Cu") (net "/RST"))
 (segment (start 54.815686 36.315686) (end 56.372028 34.759344) (width 0.2) (layer "F.Cu") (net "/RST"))
 (segment (start 95 34.42) (end 99.82 39.24) (width 0.2) (layer "F.Cu") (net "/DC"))
 (segment (start 54.4 44.21) (end 54.4 36.165686) (width 0.2) (layer "F.Cu") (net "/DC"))
 (segment (start 56.206342 34.359344) (end 95 34.359344) (width 0.2) (layer "F.Cu") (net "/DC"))
 (segment (start 63 52.81) (end 54.4 44.21) (width 0.2) (layer "F.Cu") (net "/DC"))
 (segment (start 95 34.359344) (end 95 34.42) (width 0.2) (layer "F.Cu") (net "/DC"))
 (segment (start 54.4 36.165686) (end 56.206342 34.359344) (width 0.2) (layer "F.Cu") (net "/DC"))
 (segment (start 56.7034 35.559344) (end 88.519344 35.559344) (width 0.2) (layer "F.Cu") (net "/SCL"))
 (segment (start 55.615686 37.805686) (end 55.615686 36.647058) (width 0.2) (layer "F.Cu") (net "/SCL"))
 (segment (start 63 45.19) (end 55.615686 37.805686) (width 0.2) (layer "F.Cu") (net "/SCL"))
 (segment (start 88.519344 35.559344) (end 92.2 39.24) (width 0.2) (layer "F.Cu") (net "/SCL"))
 (segment (start 55.615686 36.647058) (end 56.7034 35.559344) (width 0.2) (layer "F.Cu") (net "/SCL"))
 (segment (start 63 55.35) (end 54 46.35) (width 0.2) (layer "F.Cu") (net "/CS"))
 (segment (start 56.040656 33.959344) (end 97.079344 33.959344) (width 0.2) (layer "F.Cu") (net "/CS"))
 (segment (start 54 36) (end 56.040656 33.959344) (width 0.2) (layer "F.Cu") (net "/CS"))
 (segment (start 54 46.35) (end 54 36) (width 0.2) (layer "F.Cu") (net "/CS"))
 (segment (start 97.079344 33.959344) (end 102.36 39.24) (width 0.2) (layer "F.Cu") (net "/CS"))
 (segment (start 56.537714 35.159344) (end 90.659344 35.159344) (width 0.2) (layer "F.Cu") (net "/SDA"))
 (segment (start 90.659344 35.159344) (end 94.74 39.24) (width 0.2) (layer "F.Cu") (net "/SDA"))
 (segment (start 55.215686 39.945686) (end 55.215686 36.481372) (width 0.2) (layer "F.Cu") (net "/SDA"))
 (segment (start 63 47.73) (end 55.215686 39.945686) (width 0.2) (layer "F.Cu") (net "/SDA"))
 (segment (start 55.215686 36.481372) (end 56.537714 35.159344) (width 0.2) (layer "F.Cu") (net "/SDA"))
 (segment (start 53.5 68.4) (end 49.74 72.16) (width 0.2) (layer "F.Cu") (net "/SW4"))
 (segment (start 99.219344 33.559344) (end 55.87497 33.559344) (width 0.2) (layer "F.Cu") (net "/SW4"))
 (segment (start 55.87497 33.559344) (end 53.5 35.934314) (width 0.2) (layer "F.Cu") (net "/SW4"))
 (segment (start 53.5 35.934314) (end 53.5 68.4) (width 0.2) (layer "F.Cu") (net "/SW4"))
 (segment (start 104.9 39.24) (end 99.219344 33.559344) (width 0.2) (layer "F.Cu") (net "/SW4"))
 (segment (start 89.5 61) (end 90.5 60) (width 0.2) (layer "F.Cu") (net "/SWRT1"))
 (segment (start 89.5 63.5) (end 89.5 61) (width 0.2) (layer "F.Cu") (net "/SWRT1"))
 (segment (start 122.6 77.3) (end 121.3 78.6) (width 0.2) (layer "F.Cu") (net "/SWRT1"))
 (segment (start 90.5 60) (end 95.18 60) (width 0.2) (layer "F.Cu") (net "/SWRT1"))
 (segment (start 106.6 78.6) (end 93.5 65.5) (width 0.2) (layer "F.Cu") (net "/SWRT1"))
 (segment (start 95.18 60) (end 97.28 62.1) (width 0.2) (layer "F.Cu") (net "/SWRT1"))
 (segment (start 91.5 65.5) (end 89.5 63.5) (width 0.2) (layer "F.Cu") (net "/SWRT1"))
 (segment (start 121.3 78.6) (end 106.6 78.6) (width 0.2) (layer "F.Cu") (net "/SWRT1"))
 (segment (start 93.5 65.5) (end 91.5 65.5) (width 0.2) (layer "F.Cu") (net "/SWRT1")))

